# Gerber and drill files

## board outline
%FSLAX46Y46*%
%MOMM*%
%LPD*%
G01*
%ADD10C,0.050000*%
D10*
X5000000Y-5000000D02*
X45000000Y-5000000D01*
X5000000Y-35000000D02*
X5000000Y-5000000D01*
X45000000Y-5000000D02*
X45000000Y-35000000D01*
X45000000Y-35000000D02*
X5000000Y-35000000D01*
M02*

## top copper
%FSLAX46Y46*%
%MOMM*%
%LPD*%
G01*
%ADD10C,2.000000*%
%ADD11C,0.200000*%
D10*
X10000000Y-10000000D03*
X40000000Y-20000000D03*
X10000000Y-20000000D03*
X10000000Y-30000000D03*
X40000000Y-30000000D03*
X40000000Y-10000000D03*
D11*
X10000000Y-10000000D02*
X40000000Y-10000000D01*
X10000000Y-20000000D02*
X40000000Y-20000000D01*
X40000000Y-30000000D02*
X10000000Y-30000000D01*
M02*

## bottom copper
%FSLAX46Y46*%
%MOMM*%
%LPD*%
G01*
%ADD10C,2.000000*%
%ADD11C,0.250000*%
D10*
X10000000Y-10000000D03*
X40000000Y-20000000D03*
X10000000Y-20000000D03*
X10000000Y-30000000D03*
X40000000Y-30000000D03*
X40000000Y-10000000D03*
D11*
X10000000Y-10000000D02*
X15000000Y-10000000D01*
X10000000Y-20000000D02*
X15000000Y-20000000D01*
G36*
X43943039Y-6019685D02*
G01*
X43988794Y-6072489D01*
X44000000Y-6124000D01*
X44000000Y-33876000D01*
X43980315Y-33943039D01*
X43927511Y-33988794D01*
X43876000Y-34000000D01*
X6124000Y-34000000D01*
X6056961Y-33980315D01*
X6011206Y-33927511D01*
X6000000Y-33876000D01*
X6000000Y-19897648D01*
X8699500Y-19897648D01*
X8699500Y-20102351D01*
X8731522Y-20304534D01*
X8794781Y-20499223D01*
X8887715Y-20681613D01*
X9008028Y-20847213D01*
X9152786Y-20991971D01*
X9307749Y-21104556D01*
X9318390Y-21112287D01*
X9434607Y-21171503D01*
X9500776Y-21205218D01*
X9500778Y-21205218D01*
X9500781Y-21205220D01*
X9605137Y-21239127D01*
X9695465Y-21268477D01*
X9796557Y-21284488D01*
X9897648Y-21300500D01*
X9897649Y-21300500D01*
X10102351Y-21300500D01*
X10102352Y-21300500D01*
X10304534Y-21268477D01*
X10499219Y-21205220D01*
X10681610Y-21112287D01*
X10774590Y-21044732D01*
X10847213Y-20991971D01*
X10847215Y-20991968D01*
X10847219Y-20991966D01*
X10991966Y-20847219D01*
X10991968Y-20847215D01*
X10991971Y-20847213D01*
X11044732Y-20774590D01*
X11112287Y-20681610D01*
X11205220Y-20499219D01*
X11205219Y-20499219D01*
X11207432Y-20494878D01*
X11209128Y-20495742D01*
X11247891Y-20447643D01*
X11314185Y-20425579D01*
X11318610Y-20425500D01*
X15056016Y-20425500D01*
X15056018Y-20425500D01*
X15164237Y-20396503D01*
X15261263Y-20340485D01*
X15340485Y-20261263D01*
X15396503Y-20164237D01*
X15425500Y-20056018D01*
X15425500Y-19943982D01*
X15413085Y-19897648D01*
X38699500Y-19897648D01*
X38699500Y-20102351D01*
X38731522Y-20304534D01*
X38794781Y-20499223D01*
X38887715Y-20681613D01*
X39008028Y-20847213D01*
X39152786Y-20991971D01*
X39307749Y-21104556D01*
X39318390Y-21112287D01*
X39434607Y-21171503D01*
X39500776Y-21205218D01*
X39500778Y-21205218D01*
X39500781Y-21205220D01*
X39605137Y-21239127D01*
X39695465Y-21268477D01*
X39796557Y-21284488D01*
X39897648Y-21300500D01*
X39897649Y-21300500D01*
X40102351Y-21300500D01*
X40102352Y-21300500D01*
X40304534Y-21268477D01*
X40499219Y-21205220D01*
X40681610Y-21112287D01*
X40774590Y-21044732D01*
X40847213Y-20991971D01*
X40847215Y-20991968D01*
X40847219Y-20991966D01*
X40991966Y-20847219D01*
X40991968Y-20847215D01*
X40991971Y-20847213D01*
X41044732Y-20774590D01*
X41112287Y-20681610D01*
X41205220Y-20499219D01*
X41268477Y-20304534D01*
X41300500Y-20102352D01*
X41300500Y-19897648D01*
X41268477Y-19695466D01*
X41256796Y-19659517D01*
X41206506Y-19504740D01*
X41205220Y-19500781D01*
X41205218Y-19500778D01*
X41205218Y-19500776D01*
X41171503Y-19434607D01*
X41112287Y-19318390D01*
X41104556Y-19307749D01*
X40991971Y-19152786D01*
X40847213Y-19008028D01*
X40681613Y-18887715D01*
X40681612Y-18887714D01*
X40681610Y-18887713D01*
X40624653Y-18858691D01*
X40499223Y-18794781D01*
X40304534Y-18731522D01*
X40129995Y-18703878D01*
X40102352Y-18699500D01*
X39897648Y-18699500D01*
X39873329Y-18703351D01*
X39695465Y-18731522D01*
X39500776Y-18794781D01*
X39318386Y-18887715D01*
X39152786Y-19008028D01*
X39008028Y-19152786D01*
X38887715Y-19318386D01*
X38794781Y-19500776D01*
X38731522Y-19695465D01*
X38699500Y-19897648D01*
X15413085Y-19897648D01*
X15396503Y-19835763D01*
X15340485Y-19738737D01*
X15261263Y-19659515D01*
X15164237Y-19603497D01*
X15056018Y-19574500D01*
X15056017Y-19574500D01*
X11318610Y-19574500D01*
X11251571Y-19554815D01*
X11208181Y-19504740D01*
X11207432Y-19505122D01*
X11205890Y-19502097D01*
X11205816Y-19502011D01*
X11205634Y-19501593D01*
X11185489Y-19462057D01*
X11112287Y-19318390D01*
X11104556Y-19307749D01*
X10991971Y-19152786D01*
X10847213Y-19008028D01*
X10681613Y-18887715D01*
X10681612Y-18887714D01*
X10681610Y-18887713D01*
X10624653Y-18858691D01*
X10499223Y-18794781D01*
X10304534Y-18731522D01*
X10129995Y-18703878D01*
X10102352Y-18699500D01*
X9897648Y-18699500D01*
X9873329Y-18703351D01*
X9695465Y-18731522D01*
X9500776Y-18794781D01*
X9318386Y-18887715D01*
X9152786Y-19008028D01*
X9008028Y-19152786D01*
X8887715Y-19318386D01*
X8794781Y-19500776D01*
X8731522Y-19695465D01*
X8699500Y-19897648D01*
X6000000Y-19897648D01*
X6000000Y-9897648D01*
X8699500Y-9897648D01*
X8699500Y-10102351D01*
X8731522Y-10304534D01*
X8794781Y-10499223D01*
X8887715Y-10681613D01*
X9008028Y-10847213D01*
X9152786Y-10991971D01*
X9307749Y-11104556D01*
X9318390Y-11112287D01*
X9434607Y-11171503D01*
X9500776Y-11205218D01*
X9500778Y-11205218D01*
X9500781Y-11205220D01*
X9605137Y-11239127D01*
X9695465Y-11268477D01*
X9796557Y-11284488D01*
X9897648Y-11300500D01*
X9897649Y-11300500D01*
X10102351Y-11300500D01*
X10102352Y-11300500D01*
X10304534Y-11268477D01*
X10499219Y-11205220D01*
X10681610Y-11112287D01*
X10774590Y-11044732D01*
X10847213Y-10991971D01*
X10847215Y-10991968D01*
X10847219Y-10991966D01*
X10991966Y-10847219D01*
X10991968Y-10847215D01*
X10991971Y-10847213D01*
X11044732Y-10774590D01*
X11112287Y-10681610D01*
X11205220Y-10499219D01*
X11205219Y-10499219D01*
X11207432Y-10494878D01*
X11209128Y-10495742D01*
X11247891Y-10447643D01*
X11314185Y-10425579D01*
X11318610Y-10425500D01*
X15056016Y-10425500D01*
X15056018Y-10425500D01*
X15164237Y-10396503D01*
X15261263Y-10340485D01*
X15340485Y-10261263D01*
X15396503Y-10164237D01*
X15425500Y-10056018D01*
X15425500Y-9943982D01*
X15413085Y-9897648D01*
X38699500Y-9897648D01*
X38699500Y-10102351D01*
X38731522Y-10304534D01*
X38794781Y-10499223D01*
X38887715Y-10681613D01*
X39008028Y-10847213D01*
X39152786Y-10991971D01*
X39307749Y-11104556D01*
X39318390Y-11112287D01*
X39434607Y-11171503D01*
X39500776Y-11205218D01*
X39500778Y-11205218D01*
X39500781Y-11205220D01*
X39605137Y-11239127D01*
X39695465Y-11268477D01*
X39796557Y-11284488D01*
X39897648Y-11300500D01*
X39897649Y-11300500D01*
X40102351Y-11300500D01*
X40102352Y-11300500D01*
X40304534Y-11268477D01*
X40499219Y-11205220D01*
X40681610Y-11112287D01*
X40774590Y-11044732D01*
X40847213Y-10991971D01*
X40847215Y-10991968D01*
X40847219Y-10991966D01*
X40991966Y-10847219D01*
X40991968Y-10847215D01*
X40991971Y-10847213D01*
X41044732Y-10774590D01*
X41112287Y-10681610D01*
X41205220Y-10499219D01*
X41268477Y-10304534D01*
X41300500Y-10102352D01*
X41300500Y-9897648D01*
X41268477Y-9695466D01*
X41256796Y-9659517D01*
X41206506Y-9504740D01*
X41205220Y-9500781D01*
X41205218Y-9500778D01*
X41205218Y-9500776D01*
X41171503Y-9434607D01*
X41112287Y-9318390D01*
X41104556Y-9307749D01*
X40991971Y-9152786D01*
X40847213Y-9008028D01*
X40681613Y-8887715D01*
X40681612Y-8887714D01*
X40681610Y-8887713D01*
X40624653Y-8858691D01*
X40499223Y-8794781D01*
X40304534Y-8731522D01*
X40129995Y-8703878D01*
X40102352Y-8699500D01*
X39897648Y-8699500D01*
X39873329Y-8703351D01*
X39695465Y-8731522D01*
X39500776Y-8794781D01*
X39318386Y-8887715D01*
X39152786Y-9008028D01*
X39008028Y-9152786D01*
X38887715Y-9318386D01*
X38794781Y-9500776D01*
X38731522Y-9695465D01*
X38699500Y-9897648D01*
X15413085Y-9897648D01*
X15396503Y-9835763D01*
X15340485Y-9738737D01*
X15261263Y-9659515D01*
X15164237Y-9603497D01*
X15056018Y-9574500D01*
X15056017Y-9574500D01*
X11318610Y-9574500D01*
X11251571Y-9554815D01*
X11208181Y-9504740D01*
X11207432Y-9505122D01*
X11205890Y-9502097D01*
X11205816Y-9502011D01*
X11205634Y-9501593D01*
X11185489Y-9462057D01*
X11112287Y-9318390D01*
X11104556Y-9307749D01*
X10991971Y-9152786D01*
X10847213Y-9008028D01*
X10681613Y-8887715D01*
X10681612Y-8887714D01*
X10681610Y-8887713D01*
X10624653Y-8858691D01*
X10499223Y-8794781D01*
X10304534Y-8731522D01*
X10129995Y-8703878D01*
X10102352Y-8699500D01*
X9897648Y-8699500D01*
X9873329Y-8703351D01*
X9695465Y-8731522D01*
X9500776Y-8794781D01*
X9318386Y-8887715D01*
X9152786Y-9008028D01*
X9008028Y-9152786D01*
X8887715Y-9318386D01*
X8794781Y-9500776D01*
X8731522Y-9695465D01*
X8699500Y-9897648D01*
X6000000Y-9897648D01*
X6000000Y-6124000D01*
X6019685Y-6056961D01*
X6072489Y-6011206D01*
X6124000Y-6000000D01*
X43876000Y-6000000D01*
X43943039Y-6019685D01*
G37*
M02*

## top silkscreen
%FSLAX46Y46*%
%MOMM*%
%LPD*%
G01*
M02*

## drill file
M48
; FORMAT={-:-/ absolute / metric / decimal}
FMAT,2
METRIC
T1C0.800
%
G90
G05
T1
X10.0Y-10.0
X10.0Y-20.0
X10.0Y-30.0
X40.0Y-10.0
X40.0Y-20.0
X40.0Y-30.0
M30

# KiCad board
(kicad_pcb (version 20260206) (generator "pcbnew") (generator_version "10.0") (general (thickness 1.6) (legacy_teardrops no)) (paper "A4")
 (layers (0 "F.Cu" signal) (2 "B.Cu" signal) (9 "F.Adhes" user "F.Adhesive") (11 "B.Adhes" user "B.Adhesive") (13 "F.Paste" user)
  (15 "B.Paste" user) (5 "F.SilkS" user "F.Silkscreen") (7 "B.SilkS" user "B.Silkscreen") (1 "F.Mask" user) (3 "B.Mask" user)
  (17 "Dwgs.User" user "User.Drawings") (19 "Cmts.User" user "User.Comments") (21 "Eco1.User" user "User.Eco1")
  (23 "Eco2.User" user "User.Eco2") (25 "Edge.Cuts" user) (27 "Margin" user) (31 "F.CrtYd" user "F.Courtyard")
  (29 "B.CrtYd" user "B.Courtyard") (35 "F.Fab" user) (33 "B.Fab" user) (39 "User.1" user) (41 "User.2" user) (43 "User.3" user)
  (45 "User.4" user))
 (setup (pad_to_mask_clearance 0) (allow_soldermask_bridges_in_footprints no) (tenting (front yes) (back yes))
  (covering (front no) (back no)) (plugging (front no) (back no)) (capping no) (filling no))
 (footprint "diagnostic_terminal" (layer "F.Cu") (at 10 10)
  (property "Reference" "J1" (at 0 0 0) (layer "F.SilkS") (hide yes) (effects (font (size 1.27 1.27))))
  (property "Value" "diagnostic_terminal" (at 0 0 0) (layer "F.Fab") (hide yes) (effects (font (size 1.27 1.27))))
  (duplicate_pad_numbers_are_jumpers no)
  (pad "1" thru_hole circle (at 0 0) (size 2 2) (drill 0.8) (layers "*.Cu") (remove_unused_layers no) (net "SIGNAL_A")))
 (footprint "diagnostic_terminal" (layer "F.Cu") (at 40 20)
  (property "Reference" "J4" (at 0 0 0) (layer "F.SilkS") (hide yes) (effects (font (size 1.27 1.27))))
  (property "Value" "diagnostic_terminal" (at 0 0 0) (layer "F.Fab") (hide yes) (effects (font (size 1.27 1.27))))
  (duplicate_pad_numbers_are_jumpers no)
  (pad "1" thru_hole circle (at 0 0) (size 2 2) (drill 0.8) (layers "*.Cu") (remove_unused_layers no) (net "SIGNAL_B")))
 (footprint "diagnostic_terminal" (layer "F.Cu") (at 10 20)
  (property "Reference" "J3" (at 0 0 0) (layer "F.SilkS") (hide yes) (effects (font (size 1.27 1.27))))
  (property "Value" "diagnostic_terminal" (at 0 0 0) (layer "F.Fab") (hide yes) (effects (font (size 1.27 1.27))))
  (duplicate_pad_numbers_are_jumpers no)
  (pad "1" thru_hole circle (at 0 0) (size 2 2) (drill 0.8) (layers "*.Cu") (remove_unused_layers no) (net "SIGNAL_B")))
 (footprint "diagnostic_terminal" (layer "F.Cu") (at 10 30)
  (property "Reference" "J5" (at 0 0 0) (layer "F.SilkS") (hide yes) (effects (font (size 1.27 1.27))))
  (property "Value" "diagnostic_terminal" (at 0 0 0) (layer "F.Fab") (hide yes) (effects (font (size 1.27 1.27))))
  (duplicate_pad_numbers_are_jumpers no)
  (pad "1" thru_hole circle (at 0 0) (size 2 2) (drill 0.8) (layers "*.Cu") (remove_unused_layers no) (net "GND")))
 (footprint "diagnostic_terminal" (layer "F.Cu") (at 40 30)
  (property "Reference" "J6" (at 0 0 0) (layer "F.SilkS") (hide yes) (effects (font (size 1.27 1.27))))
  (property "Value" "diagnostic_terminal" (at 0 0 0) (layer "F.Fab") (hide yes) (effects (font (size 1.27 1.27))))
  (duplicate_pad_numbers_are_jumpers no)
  (pad "1" thru_hole circle (at 0 0) (size 2 2) (drill 0.8) (layers "*.Cu") (remove_unused_layers no) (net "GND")))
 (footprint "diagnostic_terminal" (layer "F.Cu") (at 40 10)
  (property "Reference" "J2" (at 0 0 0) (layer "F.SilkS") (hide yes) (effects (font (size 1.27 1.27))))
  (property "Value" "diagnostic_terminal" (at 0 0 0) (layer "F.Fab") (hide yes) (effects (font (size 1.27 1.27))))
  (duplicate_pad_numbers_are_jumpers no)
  (pad "1" thru_hole circle (at 0 0) (size 2 2) (drill 0.8) (layers "*.Cu") (remove_unused_layers no) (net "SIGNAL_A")))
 (gr_line (start 5 5) (end 45 5) (stroke (width 0.05) (type default)) (layer "Edge.Cuts"))
 (gr_line (start 5 35) (end 5 5) (stroke (width 0.05) (type default)) (layer "Edge.Cuts"))
 (gr_line (start 45 5) (end 45 35) (stroke (width 0.05) (type default)) (layer "Edge.Cuts"))
 (gr_line (start 45 35) (end 5 35) (stroke (width 0.05) (type default)) (layer "Edge.Cuts"))
 (segment (start 10 10) (end 40 10) (width 0.2) (layer "F.Cu") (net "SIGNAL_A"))
 (segment (start 10 10) (end 15 10) (width 0.25) (layer "B.Cu") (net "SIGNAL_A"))
 (segment (start 10 20) (end 40 20) (width 0.2) (layer "F.Cu") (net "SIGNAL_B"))
 (segment (start 10 20) (end 15 20) (width 0.25) (layer "B.Cu") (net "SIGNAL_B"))
 (segment (start 40 30) (end 10 30) (width 0.2) (layer "F.Cu") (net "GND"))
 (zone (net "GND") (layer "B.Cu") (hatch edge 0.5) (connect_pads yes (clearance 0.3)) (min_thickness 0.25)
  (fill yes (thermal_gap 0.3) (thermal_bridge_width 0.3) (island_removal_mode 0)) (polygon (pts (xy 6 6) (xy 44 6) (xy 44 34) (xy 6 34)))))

